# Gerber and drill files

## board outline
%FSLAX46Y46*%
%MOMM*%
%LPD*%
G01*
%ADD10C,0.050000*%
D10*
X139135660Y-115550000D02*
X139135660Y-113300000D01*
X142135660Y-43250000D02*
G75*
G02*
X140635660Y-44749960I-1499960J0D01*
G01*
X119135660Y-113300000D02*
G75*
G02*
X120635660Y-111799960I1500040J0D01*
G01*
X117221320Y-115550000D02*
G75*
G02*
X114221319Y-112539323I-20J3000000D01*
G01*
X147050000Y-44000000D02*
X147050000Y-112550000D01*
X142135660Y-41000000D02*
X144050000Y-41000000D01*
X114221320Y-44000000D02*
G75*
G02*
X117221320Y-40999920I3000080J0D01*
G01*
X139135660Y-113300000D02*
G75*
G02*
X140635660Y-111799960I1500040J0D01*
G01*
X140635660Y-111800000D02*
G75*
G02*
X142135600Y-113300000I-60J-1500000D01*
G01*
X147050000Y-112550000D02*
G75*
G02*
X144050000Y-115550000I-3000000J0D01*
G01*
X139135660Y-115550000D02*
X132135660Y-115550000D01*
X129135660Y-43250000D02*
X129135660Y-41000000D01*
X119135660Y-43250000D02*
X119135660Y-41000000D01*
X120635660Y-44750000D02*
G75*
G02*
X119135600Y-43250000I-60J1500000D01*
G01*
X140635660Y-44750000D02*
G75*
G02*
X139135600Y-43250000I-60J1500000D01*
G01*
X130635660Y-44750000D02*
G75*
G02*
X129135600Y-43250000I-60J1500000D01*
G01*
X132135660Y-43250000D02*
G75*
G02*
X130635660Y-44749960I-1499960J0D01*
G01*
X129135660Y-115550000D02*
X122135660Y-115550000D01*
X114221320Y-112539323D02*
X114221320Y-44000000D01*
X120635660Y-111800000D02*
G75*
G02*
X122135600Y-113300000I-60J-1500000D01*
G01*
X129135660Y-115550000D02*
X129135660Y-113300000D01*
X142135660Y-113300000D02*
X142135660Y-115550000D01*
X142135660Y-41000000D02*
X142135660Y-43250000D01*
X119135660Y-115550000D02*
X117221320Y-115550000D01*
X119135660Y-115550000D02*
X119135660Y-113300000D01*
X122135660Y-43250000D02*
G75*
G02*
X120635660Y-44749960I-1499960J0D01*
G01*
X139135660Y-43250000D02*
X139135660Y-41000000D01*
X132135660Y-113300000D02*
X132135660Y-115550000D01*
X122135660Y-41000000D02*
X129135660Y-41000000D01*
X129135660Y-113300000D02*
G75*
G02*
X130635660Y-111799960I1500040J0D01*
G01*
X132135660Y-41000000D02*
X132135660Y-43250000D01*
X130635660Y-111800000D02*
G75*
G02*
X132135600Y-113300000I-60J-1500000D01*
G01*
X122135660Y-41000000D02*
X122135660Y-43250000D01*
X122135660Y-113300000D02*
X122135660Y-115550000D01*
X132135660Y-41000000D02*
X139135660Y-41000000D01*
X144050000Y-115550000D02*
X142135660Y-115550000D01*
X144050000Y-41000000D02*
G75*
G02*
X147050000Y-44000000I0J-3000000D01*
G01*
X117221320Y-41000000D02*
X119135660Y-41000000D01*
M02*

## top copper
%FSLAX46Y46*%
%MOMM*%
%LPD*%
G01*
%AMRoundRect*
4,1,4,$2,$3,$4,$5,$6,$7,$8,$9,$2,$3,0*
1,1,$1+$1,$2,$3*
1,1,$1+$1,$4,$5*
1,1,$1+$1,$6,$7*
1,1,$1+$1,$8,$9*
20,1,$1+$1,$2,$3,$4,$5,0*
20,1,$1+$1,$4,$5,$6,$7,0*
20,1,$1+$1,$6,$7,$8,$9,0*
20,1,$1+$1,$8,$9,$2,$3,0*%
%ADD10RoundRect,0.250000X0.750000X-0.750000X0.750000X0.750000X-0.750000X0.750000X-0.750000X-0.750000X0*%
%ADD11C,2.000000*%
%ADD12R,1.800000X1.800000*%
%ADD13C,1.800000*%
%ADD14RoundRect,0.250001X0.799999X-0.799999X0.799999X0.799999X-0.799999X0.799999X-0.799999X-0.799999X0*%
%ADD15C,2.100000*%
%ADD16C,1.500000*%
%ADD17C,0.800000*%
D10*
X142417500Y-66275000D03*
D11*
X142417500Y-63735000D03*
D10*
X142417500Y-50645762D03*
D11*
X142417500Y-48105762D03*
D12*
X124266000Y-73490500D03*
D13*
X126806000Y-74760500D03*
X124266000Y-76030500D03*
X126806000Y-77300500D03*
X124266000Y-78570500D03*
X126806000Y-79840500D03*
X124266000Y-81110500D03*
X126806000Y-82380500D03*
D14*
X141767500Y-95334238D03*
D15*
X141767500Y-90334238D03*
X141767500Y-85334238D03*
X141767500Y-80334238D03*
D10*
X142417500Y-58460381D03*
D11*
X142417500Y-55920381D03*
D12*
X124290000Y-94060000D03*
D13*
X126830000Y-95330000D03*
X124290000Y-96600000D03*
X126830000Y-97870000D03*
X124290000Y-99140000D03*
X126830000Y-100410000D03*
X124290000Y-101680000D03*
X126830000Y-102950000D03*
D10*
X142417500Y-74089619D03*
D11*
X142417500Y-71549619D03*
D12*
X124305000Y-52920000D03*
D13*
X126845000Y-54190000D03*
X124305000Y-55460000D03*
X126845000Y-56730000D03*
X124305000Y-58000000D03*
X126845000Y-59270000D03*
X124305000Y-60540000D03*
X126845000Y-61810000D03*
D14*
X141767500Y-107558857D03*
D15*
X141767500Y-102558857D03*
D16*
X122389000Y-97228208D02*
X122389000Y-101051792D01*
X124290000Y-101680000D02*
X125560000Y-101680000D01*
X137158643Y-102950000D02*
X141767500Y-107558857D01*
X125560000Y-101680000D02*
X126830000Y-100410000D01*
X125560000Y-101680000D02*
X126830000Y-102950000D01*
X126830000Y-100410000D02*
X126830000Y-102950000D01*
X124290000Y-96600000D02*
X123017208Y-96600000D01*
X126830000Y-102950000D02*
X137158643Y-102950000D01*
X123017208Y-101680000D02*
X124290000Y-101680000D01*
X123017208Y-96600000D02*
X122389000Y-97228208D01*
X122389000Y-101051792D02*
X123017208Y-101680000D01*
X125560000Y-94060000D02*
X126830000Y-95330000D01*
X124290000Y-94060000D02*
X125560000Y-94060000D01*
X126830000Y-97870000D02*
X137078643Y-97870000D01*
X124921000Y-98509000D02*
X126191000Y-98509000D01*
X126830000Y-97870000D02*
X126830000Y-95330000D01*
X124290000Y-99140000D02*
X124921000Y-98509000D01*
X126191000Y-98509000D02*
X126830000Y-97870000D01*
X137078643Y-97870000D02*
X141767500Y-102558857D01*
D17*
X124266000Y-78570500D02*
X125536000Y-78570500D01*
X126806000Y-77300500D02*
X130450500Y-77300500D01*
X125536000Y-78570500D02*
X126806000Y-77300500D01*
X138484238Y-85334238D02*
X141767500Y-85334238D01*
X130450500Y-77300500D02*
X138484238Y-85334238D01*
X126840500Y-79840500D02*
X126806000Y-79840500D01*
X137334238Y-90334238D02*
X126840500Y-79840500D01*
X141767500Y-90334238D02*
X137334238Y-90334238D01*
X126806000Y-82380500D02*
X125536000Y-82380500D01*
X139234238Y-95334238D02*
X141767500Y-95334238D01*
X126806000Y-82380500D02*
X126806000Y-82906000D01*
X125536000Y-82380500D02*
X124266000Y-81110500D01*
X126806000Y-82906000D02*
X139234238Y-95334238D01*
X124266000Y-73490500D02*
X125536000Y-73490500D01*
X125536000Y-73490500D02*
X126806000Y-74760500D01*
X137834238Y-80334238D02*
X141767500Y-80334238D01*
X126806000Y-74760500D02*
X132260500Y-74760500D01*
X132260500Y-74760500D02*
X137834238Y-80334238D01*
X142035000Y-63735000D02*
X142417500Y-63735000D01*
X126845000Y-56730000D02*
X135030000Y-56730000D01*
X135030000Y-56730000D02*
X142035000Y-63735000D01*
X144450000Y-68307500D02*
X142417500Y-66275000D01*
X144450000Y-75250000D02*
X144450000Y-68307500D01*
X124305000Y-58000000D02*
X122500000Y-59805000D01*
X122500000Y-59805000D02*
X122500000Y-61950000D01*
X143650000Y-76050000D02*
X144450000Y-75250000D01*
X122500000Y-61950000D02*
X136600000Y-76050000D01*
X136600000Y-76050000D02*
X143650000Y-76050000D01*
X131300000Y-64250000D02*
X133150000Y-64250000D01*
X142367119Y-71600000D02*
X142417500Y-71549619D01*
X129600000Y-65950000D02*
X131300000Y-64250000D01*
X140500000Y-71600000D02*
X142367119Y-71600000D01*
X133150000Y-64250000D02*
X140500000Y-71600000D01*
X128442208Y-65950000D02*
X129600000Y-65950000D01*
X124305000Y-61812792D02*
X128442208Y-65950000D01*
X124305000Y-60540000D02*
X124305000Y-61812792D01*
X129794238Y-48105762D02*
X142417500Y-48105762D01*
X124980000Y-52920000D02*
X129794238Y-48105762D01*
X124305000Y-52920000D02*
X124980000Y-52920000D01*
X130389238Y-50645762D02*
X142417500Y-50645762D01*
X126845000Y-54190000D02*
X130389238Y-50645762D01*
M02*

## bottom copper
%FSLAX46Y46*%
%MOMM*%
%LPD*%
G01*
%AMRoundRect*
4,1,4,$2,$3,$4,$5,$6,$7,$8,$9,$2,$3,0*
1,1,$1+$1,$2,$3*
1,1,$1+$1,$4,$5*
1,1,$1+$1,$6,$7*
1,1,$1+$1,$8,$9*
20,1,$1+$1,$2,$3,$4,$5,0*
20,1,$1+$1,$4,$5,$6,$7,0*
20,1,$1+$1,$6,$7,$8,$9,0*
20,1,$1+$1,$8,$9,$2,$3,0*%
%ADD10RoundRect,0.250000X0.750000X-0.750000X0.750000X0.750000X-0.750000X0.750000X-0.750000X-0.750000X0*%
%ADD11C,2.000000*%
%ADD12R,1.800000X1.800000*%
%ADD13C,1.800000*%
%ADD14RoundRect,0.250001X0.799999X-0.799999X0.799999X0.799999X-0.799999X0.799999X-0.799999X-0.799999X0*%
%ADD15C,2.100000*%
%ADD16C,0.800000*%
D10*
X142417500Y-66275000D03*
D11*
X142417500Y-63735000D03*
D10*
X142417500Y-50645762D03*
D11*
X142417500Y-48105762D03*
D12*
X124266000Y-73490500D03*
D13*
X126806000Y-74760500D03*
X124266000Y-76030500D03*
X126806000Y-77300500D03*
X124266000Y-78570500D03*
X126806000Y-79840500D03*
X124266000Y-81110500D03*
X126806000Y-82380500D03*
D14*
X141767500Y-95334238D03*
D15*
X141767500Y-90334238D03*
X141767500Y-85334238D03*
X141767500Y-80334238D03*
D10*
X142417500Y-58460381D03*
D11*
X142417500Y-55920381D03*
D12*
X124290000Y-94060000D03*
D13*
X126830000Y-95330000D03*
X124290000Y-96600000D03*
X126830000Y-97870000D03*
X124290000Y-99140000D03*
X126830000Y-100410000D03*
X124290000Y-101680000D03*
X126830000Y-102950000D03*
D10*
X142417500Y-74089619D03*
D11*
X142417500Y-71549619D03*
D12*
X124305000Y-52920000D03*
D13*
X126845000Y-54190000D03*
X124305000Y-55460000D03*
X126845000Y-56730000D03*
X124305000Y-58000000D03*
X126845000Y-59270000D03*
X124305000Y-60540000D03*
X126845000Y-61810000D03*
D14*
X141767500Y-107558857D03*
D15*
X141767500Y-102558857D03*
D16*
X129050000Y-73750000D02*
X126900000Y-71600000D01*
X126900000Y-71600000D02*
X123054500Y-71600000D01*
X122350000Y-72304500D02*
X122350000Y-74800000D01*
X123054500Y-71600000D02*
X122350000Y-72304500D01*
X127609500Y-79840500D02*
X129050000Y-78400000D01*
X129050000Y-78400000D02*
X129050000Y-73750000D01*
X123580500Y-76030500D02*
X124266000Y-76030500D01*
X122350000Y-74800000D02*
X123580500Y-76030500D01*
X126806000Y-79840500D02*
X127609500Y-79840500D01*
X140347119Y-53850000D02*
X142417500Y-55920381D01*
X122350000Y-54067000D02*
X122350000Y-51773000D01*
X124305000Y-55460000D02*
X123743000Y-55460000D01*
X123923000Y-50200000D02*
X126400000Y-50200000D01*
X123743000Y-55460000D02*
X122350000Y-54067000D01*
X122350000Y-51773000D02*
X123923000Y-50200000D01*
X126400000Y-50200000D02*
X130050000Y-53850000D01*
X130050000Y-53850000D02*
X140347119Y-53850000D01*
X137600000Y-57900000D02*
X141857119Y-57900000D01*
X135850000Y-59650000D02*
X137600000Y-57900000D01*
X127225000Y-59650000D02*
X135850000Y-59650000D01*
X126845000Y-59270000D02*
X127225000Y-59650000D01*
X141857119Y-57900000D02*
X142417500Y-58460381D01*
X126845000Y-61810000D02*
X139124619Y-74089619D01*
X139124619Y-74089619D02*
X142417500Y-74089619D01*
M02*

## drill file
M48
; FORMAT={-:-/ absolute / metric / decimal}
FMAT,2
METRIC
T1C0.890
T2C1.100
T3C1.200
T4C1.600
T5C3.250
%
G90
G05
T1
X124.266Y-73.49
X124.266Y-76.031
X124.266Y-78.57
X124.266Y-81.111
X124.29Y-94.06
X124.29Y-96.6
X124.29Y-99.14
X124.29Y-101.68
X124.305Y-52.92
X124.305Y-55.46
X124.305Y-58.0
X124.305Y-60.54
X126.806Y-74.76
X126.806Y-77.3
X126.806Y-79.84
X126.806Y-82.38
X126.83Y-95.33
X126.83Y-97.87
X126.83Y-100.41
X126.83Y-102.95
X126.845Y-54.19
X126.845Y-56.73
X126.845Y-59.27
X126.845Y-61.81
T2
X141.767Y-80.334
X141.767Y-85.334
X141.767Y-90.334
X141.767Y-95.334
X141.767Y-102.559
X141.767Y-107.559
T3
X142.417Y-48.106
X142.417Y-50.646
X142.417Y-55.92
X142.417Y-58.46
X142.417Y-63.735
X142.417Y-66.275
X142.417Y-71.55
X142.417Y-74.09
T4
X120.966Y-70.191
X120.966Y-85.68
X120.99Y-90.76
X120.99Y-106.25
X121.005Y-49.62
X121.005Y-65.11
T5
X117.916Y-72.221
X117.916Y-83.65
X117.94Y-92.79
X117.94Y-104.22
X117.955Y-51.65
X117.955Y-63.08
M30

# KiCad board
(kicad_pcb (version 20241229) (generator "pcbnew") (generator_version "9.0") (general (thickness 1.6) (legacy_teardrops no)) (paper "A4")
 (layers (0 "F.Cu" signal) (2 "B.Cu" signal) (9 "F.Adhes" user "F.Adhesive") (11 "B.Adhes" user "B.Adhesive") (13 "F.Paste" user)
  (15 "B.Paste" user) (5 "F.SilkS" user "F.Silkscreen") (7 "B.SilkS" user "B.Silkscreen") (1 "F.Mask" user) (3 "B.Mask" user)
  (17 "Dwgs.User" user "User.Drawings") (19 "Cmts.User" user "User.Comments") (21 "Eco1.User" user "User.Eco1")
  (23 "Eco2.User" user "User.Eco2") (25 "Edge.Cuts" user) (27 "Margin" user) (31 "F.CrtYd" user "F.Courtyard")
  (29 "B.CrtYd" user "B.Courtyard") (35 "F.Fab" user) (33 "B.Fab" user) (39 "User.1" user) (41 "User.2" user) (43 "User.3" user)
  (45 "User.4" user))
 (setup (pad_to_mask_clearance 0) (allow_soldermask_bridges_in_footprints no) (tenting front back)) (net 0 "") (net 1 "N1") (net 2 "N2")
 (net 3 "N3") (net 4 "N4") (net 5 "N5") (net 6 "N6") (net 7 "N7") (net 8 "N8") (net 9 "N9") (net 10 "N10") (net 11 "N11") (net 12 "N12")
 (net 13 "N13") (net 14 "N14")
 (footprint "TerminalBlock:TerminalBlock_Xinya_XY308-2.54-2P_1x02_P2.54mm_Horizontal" (layer "F.Cu") (at 142.4175 66.275 90)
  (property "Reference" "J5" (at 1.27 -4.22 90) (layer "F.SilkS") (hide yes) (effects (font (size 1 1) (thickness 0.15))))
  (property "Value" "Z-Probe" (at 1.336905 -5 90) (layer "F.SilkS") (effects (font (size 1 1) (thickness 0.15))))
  (pad "1" thru_hole roundrect (at 0 0 90) (size 2 2) (drill 1.2) (layers "*.Cu" "*.Mask") (remove_unused_layers no)
   (roundrect_rratio 0.125) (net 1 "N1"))
  (pad "2" thru_hole circle (at 2.54 0 90) (size 2 2) (drill 1.2) (layers "*.Cu" "*.Mask") (remove_unused_layers no) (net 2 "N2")))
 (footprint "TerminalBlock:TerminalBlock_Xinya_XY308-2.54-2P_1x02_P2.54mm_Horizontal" (layer "F.Cu") (at 142.4175 50.645762 90)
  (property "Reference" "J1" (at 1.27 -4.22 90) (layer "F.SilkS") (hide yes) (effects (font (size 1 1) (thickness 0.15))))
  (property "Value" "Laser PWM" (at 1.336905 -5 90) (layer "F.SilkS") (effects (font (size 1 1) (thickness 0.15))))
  (pad "1" thru_hole roundrect (at 0 0 90) (size 2 2) (drill 1.2) (layers "*.Cu" "*.Mask") (remove_unused_layers no)
   (roundrect_rratio 0.125) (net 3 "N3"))
  (pad "2" thru_hole circle (at 2.54 0 90) (size 2 2) (drill 1.2) (layers "*.Cu" "*.Mask") (remove_unused_layers no) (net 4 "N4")))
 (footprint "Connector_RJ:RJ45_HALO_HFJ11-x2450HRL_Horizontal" (layer "F.Cu") (at 124.266 73.4905 -90)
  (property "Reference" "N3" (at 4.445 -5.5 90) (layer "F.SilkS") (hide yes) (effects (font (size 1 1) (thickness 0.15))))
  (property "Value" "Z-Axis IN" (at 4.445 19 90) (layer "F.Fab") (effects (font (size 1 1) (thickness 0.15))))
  (pad "" np_thru_hole circle (at -3.3 3.3 270) (size 3 3) (drill 1.6) (layers "*.Mask"))
  (pad "" np_thru_hole circle (at -1.27 6.35 270) (size 3.25 3.25) (drill 3.25) (layers "*.Cu" "*.Mask"))
  (pad "" np_thru_hole circle (at 10.16 6.35 270) (size 3.25 3.25) (drill 3.25) (layers "*.Cu" "*.Mask"))
  (pad "" np_thru_hole circle (at 12.19 3.3 270) (size 3 3) (drill 1.6) (layers "*.Mask"))
  (pad "1" thru_hole rect (at 0 0 270) (size 1.8 1.8) (drill 0.89) (layers "*.Cu" "*.Mask") (remove_unused_layers no) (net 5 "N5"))
  (pad "2" thru_hole circle (at 1.27 -2.54 270) (size 1.8 1.8) (drill 0.89) (layers "*.Cu" "*.Mask") (remove_unused_layers no) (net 5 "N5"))
  (pad "3" thru_hole circle (at 2.54 0 270) (size 1.8 1.8) (drill 0.89) (layers "*.Cu" "*.Mask") (remove_unused_layers no) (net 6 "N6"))
  (pad "4" thru_hole circle (at 3.81 -2.54 270) (size 1.8 1.8) (drill 0.89) (layers "*.Cu" "*.Mask") (remove_unused_layers no) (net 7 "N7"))
  (pad "5" thru_hole circle (at 5.08 0 270) (size 1.8 1.8) (drill 0.89) (layers "*.Cu" "*.Mask") (remove_unused_layers no) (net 7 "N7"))
  (pad "6" thru_hole circle (at 6.35 -2.54 270) (size 1.8 1.8) (drill 0.89) (layers "*.Cu" "*.Mask") (remove_unused_layers no) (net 6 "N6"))
  (pad "7" thru_hole circle (at 7.62 0 270) (size 1.8 1.8) (drill 0.89) (layers "*.Cu" "*.Mask") (remove_unused_layers no) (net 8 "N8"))
  (pad "8" thru_hole circle (at 8.89 -2.54 270) (size 1.8 1.8) (drill 0.89) (layers "*.Cu" "*.Mask") (remove_unused_layers no) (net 8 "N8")))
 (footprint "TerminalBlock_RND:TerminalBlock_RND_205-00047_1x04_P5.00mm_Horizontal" (layer "F.Cu") (at 141.7675 95.334238 90)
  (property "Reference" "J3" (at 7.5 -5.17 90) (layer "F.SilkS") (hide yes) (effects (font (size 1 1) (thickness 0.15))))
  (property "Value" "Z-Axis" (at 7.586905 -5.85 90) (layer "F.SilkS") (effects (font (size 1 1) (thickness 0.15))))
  (pad "1" thru_hole roundrect (at 0 0 90) (size 2.1 2.1) (drill 1.1) (layers "*.Cu" "*.Mask") (remove_unused_layers no)
   (roundrect_rratio 0.119048) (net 8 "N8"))
  (pad "2" thru_hole circle (at 5 0 90) (size 2.1 2.1) (drill 1.1) (layers "*.Cu" "*.Mask") (remove_unused_layers no) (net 6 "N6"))
  (pad "3" thru_hole circle (at 10 0 90) (size 2.1 2.1) (drill 1.1) (layers "*.Cu" "*.Mask") (remove_unused_layers no) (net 7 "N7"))
  (pad "4" thru_hole circle (at 15 0 90) (size 2.1 2.1) (drill 1.1) (layers "*.Cu" "*.Mask") (remove_unused_layers no) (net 5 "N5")))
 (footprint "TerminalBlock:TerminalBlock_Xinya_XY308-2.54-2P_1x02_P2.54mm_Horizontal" (layer "F.Cu") (at 142.4175 58.460381 90)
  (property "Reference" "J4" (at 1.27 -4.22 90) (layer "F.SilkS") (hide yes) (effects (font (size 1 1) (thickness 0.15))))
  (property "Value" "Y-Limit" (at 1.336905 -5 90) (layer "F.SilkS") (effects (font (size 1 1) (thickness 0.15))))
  (pad "1" thru_hole roundrect (at 0 0 90) (size 2 2) (drill 1.2) (layers "*.Cu" "*.Mask") (remove_unused_layers no)
   (roundrect_rratio 0.125) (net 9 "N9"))
  (pad "2" thru_hole circle (at 2.54 0 90) (size 2 2) (drill 1.2) (layers "*.Cu" "*.Mask") (remove_unused_layers no) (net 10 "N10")))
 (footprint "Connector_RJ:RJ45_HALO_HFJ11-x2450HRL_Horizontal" (layer "F.Cu") (at 124.29 94.06 -90)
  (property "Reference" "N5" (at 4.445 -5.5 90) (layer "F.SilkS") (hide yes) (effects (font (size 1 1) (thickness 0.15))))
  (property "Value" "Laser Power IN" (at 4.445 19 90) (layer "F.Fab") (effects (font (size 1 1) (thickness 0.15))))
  (pad "" np_thru_hole circle (at -3.3 3.3 270) (size 3 3) (drill 1.6) (layers "*.Mask"))
  (pad "" np_thru_hole circle (at -1.27 6.35 270) (size 3.25 3.25) (drill 3.25) (layers "*.Cu" "*.Mask"))
  (pad "" np_thru_hole circle (at 10.16 6.35 270) (size 3.25 3.25) (drill 3.25) (layers "*.Cu" "*.Mask"))
  (pad "" np_thru_hole circle (at 12.19 3.3 270) (size 3 3) (drill 1.6) (layers "*.Mask"))
  (pad "1" thru_hole rect (at 0 0 270) (size 1.8 1.8) (drill 0.89) (layers "*.Cu" "*.Mask") (remove_unused_layers no) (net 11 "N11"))
  (pad "2" thru_hole circle (at 1.27 -2.54 270) (size 1.8 1.8) (drill 0.89) (layers "*.Cu" "*.Mask") (remove_unused_layers no)
   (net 11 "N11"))
  (pad "3" thru_hole circle (at 2.54 0 270) (size 1.8 1.8) (drill 0.89) (layers "*.Cu" "*.Mask") (remove_unused_layers no) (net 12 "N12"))
  (pad "4" thru_hole circle (at 3.81 -2.54 270) (size 1.8 1.8) (drill 0.89) (layers "*.Cu" "*.Mask") (remove_unused_layers no)
   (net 11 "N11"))
  (pad "5" thru_hole circle (at 5.08 0 270) (size 1.8 1.8) (drill 0.89) (layers "*.Cu" "*.Mask") (remove_unused_layers no) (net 11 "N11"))
  (pad "6" thru_hole circle (at 6.35 -2.54 270) (size 1.8 1.8) (drill 0.89) (layers "*.Cu" "*.Mask") (remove_unused_layers no)
   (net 12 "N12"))
  (pad "7" thru_hole circle (at 7.62 0 270) (size 1.8 1.8) (drill 0.89) (layers "*.Cu" "*.Mask") (remove_unused_layers no) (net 12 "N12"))
  (pad "8" thru_hole circle (at 8.89 -2.54 270) (size 1.8 1.8) (drill 0.89) (layers "*.Cu" "*.Mask") (remove_unused_layers no)
   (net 12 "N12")))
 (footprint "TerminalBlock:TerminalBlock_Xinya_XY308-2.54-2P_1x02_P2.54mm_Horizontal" (layer "F.Cu") (at 142.4175 74.089619 90)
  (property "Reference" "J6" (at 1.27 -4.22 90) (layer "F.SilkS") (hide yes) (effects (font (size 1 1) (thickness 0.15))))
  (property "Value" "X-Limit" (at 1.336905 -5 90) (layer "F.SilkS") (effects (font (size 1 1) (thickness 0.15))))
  (pad "1" thru_hole roundrect (at 0 0 90) (size 2 2) (drill 1.2) (layers "*.Cu" "*.Mask") (remove_unused_layers no)
   (roundrect_rratio 0.125) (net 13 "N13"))
  (pad "2" thru_hole circle (at 2.54 0 90) (size 2 2) (drill 1.2) (layers "*.Cu" "*.Mask") (remove_unused_layers no) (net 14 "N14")))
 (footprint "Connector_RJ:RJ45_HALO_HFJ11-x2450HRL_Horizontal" (layer "F.Cu") (at 124.305 52.92 -90)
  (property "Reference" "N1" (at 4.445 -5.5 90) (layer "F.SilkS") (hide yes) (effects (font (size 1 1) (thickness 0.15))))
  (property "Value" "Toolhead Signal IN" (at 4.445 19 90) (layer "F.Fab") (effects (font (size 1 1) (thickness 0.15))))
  (pad "" np_thru_hole circle (at -3.3 3.3 270) (size 3 3) (drill 1.6) (layers "*.Mask"))
  (pad "" np_thru_hole circle (at -1.27 6.35 270) (size 3.25 3.25) (drill 3.25) (layers "*.Cu" "*.Mask"))
  (pad "" np_thru_hole circle (at 10.16 6.35 270) (size 3.25 3.25) (drill 3.25) (layers "*.Cu" "*.Mask"))
  (pad "" np_thru_hole circle (at 12.19 3.3 270) (size 3 3) (drill 1.6) (layers "*.Mask"))
  (pad "1" thru_hole rect (at 0 0 270) (size 1.8 1.8) (drill 0.89) (layers "*.Cu" "*.Mask") (remove_unused_layers no) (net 4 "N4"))
  (pad "2" thru_hole circle (at 1.27 -2.54 270) (size 1.8 1.8) (drill 0.89) (layers "*.Cu" "*.Mask") (remove_unused_layers no) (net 3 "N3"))
  (pad "3" thru_hole circle (at 2.54 0 270) (size 1.8 1.8) (drill 0.89) (layers "*.Cu" "*.Mask") (remove_unused_layers no) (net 10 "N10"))
  (pad "4" thru_hole circle (at 3.81 -2.54 270) (size 1.8 1.8) (drill 0.89) (layers "*.Cu" "*.Mask") (remove_unused_layers no) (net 2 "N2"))
  (pad "5" thru_hole circle (at 5.08 0 270) (size 1.8 1.8) (drill 0.89) (layers "*.Cu" "*.Mask") (remove_unused_layers no) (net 1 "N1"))
  (pad "6" thru_hole circle (at 6.35 -2.54 270) (size 1.8 1.8) (drill 0.89) (layers "*.Cu" "*.Mask") (remove_unused_layers no) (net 9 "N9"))
  (pad "7" thru_hole circle (at 7.62 0 270) (size 1.8 1.8) (drill 0.89) (layers "*.Cu" "*.Mask") (remove_unused_layers no) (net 14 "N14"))
  (pad "8" thru_hole circle (at 8.89 -2.54 270) (size 1.8 1.8) (drill 0.89) (layers "*.Cu" "*.Mask") (remove_unused_layers no)
   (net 13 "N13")))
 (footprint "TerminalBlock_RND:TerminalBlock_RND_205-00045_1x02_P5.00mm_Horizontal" (layer "F.Cu") (at 141.7675 107.558857 90)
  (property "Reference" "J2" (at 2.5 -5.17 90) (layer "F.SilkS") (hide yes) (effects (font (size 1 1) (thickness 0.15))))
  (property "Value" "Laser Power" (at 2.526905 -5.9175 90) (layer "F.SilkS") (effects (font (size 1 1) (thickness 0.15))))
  (pad "1" thru_hole roundrect (at 0 0 90) (size 2.1 2.1) (drill 1.1) (layers "*.Cu" "*.Mask") (remove_unused_layers no)
   (roundrect_rratio 0.119048) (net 12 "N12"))
  (pad "2" thru_hole circle (at 5 0 90) (size 2.1 2.1) (drill 1.1) (layers "*.Cu" "*.Mask") (remove_unused_layers no) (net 11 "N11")))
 (gr_line (start 139.13566 115.55) (end 139.13566 113.3) (stroke (width 0.05) (type solid)) (layer "Edge.Cuts"))
 (gr_arc (start 142.13566 43.25) (mid 141.696328 44.31068) (end 140.63566 44.75) (stroke (width 0.05) (type default)) (layer "Edge.Cuts"))
 (gr_arc (start 119.13566 113.3) (mid 119.575008 112.23936) (end 120.63566 111.8) (stroke (width 0.05) (type default)) (layer "Edge.Cuts"))
 (gr_arc (start 117.22132 115.55) (mid 115.099994 114.671326) (end 114.22132 112.539323) (stroke (width 0.05) (type default))
  (layer "Edge.Cuts"))
 (gr_line (start 147.05 44) (end 147.05 112.55) (stroke (width 0.05) (type default)) (layer "Edge.Cuts"))
 (gr_line (start 142.13566 41) (end 144.05 41) (stroke (width 0.05) (type default)) (layer "Edge.Cuts"))
 (gr_arc (start 114.22132 44) (mid 115.100008 41.8787) (end 117.22132 41) (stroke (width 0.05) (type default)) (layer "Edge.Cuts"))
 (gr_arc (start 139.13566 113.3) (mid 139.575008 112.23936) (end 140.63566 111.8) (stroke (width 0.05) (type default)) (layer "Edge.Cuts"))
 (gr_arc (start 140.63566 111.8) (mid 141.696314 112.239346) (end 142.13566 113.3) (stroke (width 0.05) (type default)) (layer "Edge.Cuts"))
 (gr_arc (start 147.05 112.55) (mid 146.171329 114.67134) (end 144.05 115.55) (stroke (width 0.05) (type default)) (layer "Edge.Cuts"))
 (gr_line (start 139.13566 115.55) (end 132.13566 115.55) (stroke (width 0.05) (type default)) (layer "Edge.Cuts"))
 (gr_line (start 129.13566 43.25) (end 129.13566 41) (stroke (width 0.05) (type solid)) (layer "Edge.Cuts"))
 (gr_line (start 119.13566 43.25) (end 119.13566 41) (stroke (width 0.05) (type solid)) (layer "Edge.Cuts"))
 (gr_arc (start 120.63566 44.75) (mid 119.574994 44.310666) (end 119.13566 43.25) (stroke (width 0.05) (type default)) (layer "Edge.Cuts"))
 (gr_arc (start 140.63566 44.75) (mid 139.574994 44.310666) (end 139.13566 43.25) (stroke (width 0.05) (type default)) (layer "Edge.Cuts"))
 (gr_arc (start 130.63566 44.75) (mid 129.574994 44.310666) (end 129.13566 43.25) (stroke (width 0.05) (type default)) (layer "Edge.Cuts"))
 (gr_arc (start 132.13566 43.25) (mid 131.696328 44.31068) (end 130.63566 44.75) (stroke (width 0.05) (type default)) (layer "Edge.Cuts"))
 (gr_line (start 129.13566 115.55) (end 122.13566 115.55) (stroke (width 0.05) (type default)) (layer "Edge.Cuts"))
 (gr_line (start 114.22132 112.539323) (end 114.22132 44) (stroke (width 0.05) (type default)) (layer "Edge.Cuts"))
 (gr_arc (start 120.63566 111.8) (mid 121.696314 112.239346) (end 122.13566 113.3) (stroke (width 0.05) (type default)) (layer "Edge.Cuts"))
 (gr_line (start 129.13566 115.55) (end 129.13566 113.3) (stroke (width 0.05) (type solid)) (layer "Edge.Cuts"))
 (gr_line (start 142.13566 113.3) (end 142.13566 115.55) (stroke (width 0.05) (type solid)) (layer "Edge.Cuts"))
 (gr_line (start 142.13566 41) (end 142.13566 43.25) (stroke (width 0.05) (type solid)) (layer "Edge.Cuts"))
 (gr_line (start 119.13566 115.55) (end 117.22132 115.55) (stroke (width 0.05) (type default)) (layer "Edge.Cuts"))
 (gr_line (start 119.13566 115.55) (end 119.13566 113.3) (stroke (width 0.05) (type solid)) (layer "Edge.Cuts"))
 (gr_arc (start 122.13566 43.25) (mid 121.696328 44.31068) (end 120.63566 44.75) (stroke (width 0.05) (type default)) (layer "Edge.Cuts"))
 (gr_line (start 139.13566 43.25) (end 139.13566 41) (stroke (width 0.05) (type solid)) (layer "Edge.Cuts"))
 (gr_line (start 132.13566 113.3) (end 132.13566 115.55) (stroke (width 0.05) (type solid)) (layer "Edge.Cuts"))
 (gr_line (start 122.13566 41) (end 129.13566 41) (stroke (width 0.05) (type default)) (layer "Edge.Cuts"))
 (gr_arc (start 129.13566 113.3) (mid 129.575008 112.23936) (end 130.63566 111.8) (stroke (width 0.05) (type default)) (layer "Edge.Cuts"))
 (gr_line (start 132.13566 41) (end 132.13566 43.25) (stroke (width 0.05) (type solid)) (layer "Edge.Cuts"))
 (gr_arc (start 130.63566 111.8) (mid 131.696314 112.239346) (end 132.13566 113.3) (stroke (width 0.05) (type default)) (layer "Edge.Cuts"))
 (gr_line (start 122.13566 41) (end 122.13566 43.25) (stroke (width 0.05) (type solid)) (layer "Edge.Cuts"))
 (gr_line (start 122.13566 113.3) (end 122.13566 115.55) (stroke (width 0.05) (type solid)) (layer "Edge.Cuts"))
 (gr_line (start 132.13566 41) (end 139.13566 41) (stroke (width 0.05) (type default)) (layer "Edge.Cuts"))
 (gr_line (start 144.05 115.55) (end 142.13566 115.55) (stroke (width 0.05) (type default)) (layer "Edge.Cuts"))
 (gr_arc (start 144.05 41) (mid 146.171314 41.878686) (end 147.05 44) (stroke (width 0.05) (type default)) (layer "Edge.Cuts"))
 (gr_line (start 117.22132 41) (end 119.13566 41) (stroke (width 0.05) (type default)) (layer "Edge.Cuts"))
 (segment (start 122.389 97.228208) (end 122.389 101.051792) (width 1.5) (layer "F.Cu") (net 12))
 (segment (start 124.29 101.68) (end 125.56 101.68) (width 1.5) (layer "F.Cu") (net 12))
 (segment (start 137.158643 102.95) (end 141.7675 107.558857) (width 1.5) (layer "F.Cu") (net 12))
 (segment (start 125.56 101.68) (end 126.83 100.41) (width 1.5) (layer "F.Cu") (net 12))
 (segment (start 125.56 101.68) (end 126.83 102.95) (width 1.5) (layer "F.Cu") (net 12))
 (segment (start 126.83 100.41) (end 126.83 102.95) (width 1.5) (layer "F.Cu") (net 12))
 (segment (start 124.29 96.6) (end 123.017208 96.6) (width 1.5) (layer "F.Cu") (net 12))
 (segment (start 126.83 102.95) (end 137.158643 102.95) (width 1.5) (layer "F.Cu") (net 12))
 (segment (start 123.017208 101.68) (end 124.29 101.68) (width 1.5) (layer "F.Cu") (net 12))
 (segment (start 123.017208 96.6) (end 122.389 97.228208) (width 1.5) (layer "F.Cu") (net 12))
 (segment (start 122.389 101.051792) (end 123.017208 101.68) (width 1.5) (layer "F.Cu") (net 12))
 (segment (start 125.56 94.06) (end 126.83 95.33) (width 1.5) (layer "F.Cu") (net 11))
 (segment (start 124.29 94.06) (end 125.56 94.06) (width 1.5) (layer "F.Cu") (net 11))
 (segment (start 126.83 97.87) (end 137.078643 97.87) (width 1.5) (layer "F.Cu") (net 11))
 (segment (start 124.921 98.509) (end 126.191 98.509) (width 1.5) (layer "F.Cu") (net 11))
 (segment (start 126.83 97.87) (end 126.83 95.33) (width 1.5) (layer "F.Cu") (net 11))
 (segment (start 124.29 99.14) (end 124.921 98.509) (width 1.5) (layer "F.Cu") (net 11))
 (segment (start 126.191 98.509) (end 126.83 97.87) (width 1.5) (layer "F.Cu") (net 11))
 (segment (start 137.078643 97.87) (end 141.7675 102.558857) (width 1.5) (layer "F.Cu") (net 11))
 (segment (start 124.266 78.5705) (end 125.536 78.5705) (width 0.8) (layer "F.Cu") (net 7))
 (segment (start 126.806 77.3005) (end 130.4505 77.3005) (width 0.8) (layer "F.Cu") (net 7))
 (segment (start 125.536 78.5705) (end 126.806 77.3005) (width 0.8) (layer "F.Cu") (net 7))
 (segment (start 138.484238 85.334238) (end 141.7675 85.334238) (width 0.8) (layer "F.Cu") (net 7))
 (segment (start 130.4505 77.3005) (end 138.484238 85.334238) (width 0.8) (layer "F.Cu") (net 7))
 (segment (start 126.8405 79.8405) (end 126.806 79.8405) (width 0.8) (layer "F.Cu") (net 6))
 (segment (start 137.334238 90.334238) (end 126.8405 79.8405) (width 0.8) (layer "F.Cu") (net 6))
 (segment (start 141.7675 90.334238) (end 137.334238 90.334238) (width 0.8) (layer "F.Cu") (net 6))
 (segment (start 129.05 73.75) (end 126.9 71.6) (width 0.8) (layer "B.Cu") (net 6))
 (segment (start 126.9 71.6) (end 123.0545 71.6) (width 0.8) (layer "B.Cu") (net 6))
 (segment (start 122.35 72.3045) (end 122.35 74.8) (width 0.8) (layer "B.Cu") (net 6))
 (segment (start 123.0545 71.6) (end 122.35 72.3045) (width 0.8) (layer "B.Cu") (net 6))
 (segment (start 127.6095 79.8405) (end 129.05 78.4) (width 0.8) (layer "B.Cu") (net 6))
 (segment (start 129.05 78.4) (end 129.05 73.75) (width 0.8) (layer "B.Cu") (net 6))
 (segment (start 123.5805 76.0305) (end 124.266 76.0305) (width 0.8) (layer "B.Cu") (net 6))
 (segment (start 122.35 74.8) (end 123.5805 76.0305) (width 0.8) (layer "B.Cu") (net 6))
 (segment (start 126.806 79.8405) (end 127.6095 79.8405) (width 0.8) (layer "B.Cu") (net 6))
 (segment (start 126.806 82.3805) (end 125.536 82.3805) (width 0.8) (layer "F.Cu") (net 8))
 (segment (start 139.234238 95.334238) (end 141.7675 95.334238) (width 0.8) (layer "F.Cu") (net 8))
 (segment (start 126.806 82.3805) (end 126.806 82.906) (width 0.8) (layer "F.Cu") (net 8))
 (segment (start 125.536 82.3805) (end 124.266 81.1105) (width 0.8) (layer "F.Cu") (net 8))
 (segment (start 126.806 82.906) (end 139.234238 95.334238) (width 0.8) (layer "F.Cu") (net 8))
 (segment (start 124.266 73.4905) (end 125.536 73.4905) (width 0.8) (layer "F.Cu") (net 5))
 (segment (start 125.536 73.4905) (end 126.806 74.7605) (width 0.8) (layer "F.Cu") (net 5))
 (segment (start 137.834238 80.334238) (end 141.7675 80.334238) (width 0.8) (layer "F.Cu") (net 5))
 (segment (start 126.806 74.7605) (end 132.2605 74.7605) (width 0.8) (layer "F.Cu") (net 5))
 (segment (start 132.2605 74.7605) (end 137.834238 80.334238) (width 0.8) (layer "F.Cu") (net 5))
 (segment (start 140.347119 53.85) (end 142.4175 55.920381) (width 0.8) (layer "B.Cu") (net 10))
 (segment (start 122.35 54.067) (end 122.35 51.773) (width 0.8) (layer "B.Cu") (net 10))
 (segment (start 124.305 55.46) (end 123.743 55.46) (width 0.8) (layer "B.Cu") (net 10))
 (segment (start 123.923 50.2) (end 126.4 50.2) (width 0.8) (layer "B.Cu") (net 10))
 (segment (start 123.743 55.46) (end 122.35 54.067) (width 0.8) (layer "B.Cu") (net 10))
 (segment (start 122.35 51.773) (end 123.923 50.2) (width 0.8) (layer "B.Cu") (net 10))
 (segment (start 126.4 50.2) (end 130.05 53.85) (width 0.8) (layer "B.Cu") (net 10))
 (segment (start 130.05 53.85) (end 140.347119 53.85) (width 0.8) (layer "B.Cu") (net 10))
 (segment (start 137.6 57.9) (end 141.857119 57.9) (width 0.8) (layer "B.Cu") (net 9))
 (segment (start 135.85 59.65) (end 137.6 57.9) (width 0.8) (layer "B.Cu") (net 9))
 (segment (start 127.225 59.65) (end 135.85 59.65) (width 0.8) (layer "B.Cu") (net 9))
 (segment (start 126.845 59.27) (end 127.225 59.65) (width 0.8) (layer "B.Cu") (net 9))
 (segment (start 141.857119 57.9) (end 142.4175 58.460381) (width 0.8) (layer "B.Cu") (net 9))
 (segment (start 142.035 63.735) (end 142.4175 63.735) (width 0.8) (layer "F.Cu") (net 2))
 (segment (start 126.845 56.73) (end 135.03 56.73) (width 0.8) (layer "F.Cu") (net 2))
 (segment (start 135.03 56.73) (end 142.035 63.735) (width 0.8) (layer "F.Cu") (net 2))
 (segment (start 144.45 68.3075) (end 142.4175 66.275) (width 0.8) (layer "F.Cu") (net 1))
 (segment (start 144.45 75.25) (end 144.45 68.3075) (width 0.8) (layer "F.Cu") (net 1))
 (segment (start 124.305 58) (end 122.5 59.805) (width 0.8) (layer "F.Cu") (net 1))
 (segment (start 122.5 59.805) (end 122.5 61.95) (width 0.8) (layer "F.Cu") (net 1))
 (segment (start 143.65 76.05) (end 144.45 75.25) (width 0.8) (layer "F.Cu") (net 1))
 (segment (start 122.5 61.95) (end 136.6 76.05) (width 0.8) (layer "F.Cu") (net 1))
 (segment (start 136.6 76.05) (end 143.65 76.05) (width 0.8) (layer "F.Cu") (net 1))
 (segment (start 131.3 64.25) (end 133.15 64.25) (width 0.8) (layer "F.Cu") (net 14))
 (segment (start 142.367119 71.6) (end 142.4175 71.549619) (width 0.8) (layer "F.Cu") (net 14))
 (segment (start 129.6 65.95) (end 131.3 64.25) (width 0.8) (layer "F.Cu") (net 14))
 (segment (start 140.5 71.6) (end 142.367119 71.6) (width 0.8) (layer "F.Cu") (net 14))
 (segment (start 133.15 64.25) (end 140.5 71.6) (width 0.8) (layer "F.Cu") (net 14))
 (segment (start 128.442208 65.95) (end 129.6 65.95) (width 0.8) (layer "F.Cu") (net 14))
 (segment (start 124.305 61.812792) (end 128.442208 65.95) (width 0.8) (layer "F.Cu") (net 14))
 (segment (start 124.305 60.54) (end 124.305 61.812792) (width 0.8) (layer "F.Cu") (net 14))
 (segment (start 129.794238 48.105762) (end 142.4175 48.105762) (width 0.8) (layer "F.Cu") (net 4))
 (segment (start 124.98 52.92) (end 129.794238 48.105762) (width 0.8) (layer "F.Cu") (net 4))
 (segment (start 124.305 52.92) (end 124.98 52.92) (width 0.8) (layer "F.Cu") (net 4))
 (segment (start 126.845 61.81) (end 139.124619 74.089619) (width 0.8) (layer "B.Cu") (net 13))
 (segment (start 139.124619 74.089619) (end 142.4175 74.089619) (width 0.8) (layer "B.Cu") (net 13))
 (segment (start 130.389238 50.645762) (end 142.4175 50.645762) (width 0.8) (layer "F.Cu") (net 3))
 (segment (start 126.845 54.19) (end 130.389238 50.645762) (width 0.8) (layer "F.Cu") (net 3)))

